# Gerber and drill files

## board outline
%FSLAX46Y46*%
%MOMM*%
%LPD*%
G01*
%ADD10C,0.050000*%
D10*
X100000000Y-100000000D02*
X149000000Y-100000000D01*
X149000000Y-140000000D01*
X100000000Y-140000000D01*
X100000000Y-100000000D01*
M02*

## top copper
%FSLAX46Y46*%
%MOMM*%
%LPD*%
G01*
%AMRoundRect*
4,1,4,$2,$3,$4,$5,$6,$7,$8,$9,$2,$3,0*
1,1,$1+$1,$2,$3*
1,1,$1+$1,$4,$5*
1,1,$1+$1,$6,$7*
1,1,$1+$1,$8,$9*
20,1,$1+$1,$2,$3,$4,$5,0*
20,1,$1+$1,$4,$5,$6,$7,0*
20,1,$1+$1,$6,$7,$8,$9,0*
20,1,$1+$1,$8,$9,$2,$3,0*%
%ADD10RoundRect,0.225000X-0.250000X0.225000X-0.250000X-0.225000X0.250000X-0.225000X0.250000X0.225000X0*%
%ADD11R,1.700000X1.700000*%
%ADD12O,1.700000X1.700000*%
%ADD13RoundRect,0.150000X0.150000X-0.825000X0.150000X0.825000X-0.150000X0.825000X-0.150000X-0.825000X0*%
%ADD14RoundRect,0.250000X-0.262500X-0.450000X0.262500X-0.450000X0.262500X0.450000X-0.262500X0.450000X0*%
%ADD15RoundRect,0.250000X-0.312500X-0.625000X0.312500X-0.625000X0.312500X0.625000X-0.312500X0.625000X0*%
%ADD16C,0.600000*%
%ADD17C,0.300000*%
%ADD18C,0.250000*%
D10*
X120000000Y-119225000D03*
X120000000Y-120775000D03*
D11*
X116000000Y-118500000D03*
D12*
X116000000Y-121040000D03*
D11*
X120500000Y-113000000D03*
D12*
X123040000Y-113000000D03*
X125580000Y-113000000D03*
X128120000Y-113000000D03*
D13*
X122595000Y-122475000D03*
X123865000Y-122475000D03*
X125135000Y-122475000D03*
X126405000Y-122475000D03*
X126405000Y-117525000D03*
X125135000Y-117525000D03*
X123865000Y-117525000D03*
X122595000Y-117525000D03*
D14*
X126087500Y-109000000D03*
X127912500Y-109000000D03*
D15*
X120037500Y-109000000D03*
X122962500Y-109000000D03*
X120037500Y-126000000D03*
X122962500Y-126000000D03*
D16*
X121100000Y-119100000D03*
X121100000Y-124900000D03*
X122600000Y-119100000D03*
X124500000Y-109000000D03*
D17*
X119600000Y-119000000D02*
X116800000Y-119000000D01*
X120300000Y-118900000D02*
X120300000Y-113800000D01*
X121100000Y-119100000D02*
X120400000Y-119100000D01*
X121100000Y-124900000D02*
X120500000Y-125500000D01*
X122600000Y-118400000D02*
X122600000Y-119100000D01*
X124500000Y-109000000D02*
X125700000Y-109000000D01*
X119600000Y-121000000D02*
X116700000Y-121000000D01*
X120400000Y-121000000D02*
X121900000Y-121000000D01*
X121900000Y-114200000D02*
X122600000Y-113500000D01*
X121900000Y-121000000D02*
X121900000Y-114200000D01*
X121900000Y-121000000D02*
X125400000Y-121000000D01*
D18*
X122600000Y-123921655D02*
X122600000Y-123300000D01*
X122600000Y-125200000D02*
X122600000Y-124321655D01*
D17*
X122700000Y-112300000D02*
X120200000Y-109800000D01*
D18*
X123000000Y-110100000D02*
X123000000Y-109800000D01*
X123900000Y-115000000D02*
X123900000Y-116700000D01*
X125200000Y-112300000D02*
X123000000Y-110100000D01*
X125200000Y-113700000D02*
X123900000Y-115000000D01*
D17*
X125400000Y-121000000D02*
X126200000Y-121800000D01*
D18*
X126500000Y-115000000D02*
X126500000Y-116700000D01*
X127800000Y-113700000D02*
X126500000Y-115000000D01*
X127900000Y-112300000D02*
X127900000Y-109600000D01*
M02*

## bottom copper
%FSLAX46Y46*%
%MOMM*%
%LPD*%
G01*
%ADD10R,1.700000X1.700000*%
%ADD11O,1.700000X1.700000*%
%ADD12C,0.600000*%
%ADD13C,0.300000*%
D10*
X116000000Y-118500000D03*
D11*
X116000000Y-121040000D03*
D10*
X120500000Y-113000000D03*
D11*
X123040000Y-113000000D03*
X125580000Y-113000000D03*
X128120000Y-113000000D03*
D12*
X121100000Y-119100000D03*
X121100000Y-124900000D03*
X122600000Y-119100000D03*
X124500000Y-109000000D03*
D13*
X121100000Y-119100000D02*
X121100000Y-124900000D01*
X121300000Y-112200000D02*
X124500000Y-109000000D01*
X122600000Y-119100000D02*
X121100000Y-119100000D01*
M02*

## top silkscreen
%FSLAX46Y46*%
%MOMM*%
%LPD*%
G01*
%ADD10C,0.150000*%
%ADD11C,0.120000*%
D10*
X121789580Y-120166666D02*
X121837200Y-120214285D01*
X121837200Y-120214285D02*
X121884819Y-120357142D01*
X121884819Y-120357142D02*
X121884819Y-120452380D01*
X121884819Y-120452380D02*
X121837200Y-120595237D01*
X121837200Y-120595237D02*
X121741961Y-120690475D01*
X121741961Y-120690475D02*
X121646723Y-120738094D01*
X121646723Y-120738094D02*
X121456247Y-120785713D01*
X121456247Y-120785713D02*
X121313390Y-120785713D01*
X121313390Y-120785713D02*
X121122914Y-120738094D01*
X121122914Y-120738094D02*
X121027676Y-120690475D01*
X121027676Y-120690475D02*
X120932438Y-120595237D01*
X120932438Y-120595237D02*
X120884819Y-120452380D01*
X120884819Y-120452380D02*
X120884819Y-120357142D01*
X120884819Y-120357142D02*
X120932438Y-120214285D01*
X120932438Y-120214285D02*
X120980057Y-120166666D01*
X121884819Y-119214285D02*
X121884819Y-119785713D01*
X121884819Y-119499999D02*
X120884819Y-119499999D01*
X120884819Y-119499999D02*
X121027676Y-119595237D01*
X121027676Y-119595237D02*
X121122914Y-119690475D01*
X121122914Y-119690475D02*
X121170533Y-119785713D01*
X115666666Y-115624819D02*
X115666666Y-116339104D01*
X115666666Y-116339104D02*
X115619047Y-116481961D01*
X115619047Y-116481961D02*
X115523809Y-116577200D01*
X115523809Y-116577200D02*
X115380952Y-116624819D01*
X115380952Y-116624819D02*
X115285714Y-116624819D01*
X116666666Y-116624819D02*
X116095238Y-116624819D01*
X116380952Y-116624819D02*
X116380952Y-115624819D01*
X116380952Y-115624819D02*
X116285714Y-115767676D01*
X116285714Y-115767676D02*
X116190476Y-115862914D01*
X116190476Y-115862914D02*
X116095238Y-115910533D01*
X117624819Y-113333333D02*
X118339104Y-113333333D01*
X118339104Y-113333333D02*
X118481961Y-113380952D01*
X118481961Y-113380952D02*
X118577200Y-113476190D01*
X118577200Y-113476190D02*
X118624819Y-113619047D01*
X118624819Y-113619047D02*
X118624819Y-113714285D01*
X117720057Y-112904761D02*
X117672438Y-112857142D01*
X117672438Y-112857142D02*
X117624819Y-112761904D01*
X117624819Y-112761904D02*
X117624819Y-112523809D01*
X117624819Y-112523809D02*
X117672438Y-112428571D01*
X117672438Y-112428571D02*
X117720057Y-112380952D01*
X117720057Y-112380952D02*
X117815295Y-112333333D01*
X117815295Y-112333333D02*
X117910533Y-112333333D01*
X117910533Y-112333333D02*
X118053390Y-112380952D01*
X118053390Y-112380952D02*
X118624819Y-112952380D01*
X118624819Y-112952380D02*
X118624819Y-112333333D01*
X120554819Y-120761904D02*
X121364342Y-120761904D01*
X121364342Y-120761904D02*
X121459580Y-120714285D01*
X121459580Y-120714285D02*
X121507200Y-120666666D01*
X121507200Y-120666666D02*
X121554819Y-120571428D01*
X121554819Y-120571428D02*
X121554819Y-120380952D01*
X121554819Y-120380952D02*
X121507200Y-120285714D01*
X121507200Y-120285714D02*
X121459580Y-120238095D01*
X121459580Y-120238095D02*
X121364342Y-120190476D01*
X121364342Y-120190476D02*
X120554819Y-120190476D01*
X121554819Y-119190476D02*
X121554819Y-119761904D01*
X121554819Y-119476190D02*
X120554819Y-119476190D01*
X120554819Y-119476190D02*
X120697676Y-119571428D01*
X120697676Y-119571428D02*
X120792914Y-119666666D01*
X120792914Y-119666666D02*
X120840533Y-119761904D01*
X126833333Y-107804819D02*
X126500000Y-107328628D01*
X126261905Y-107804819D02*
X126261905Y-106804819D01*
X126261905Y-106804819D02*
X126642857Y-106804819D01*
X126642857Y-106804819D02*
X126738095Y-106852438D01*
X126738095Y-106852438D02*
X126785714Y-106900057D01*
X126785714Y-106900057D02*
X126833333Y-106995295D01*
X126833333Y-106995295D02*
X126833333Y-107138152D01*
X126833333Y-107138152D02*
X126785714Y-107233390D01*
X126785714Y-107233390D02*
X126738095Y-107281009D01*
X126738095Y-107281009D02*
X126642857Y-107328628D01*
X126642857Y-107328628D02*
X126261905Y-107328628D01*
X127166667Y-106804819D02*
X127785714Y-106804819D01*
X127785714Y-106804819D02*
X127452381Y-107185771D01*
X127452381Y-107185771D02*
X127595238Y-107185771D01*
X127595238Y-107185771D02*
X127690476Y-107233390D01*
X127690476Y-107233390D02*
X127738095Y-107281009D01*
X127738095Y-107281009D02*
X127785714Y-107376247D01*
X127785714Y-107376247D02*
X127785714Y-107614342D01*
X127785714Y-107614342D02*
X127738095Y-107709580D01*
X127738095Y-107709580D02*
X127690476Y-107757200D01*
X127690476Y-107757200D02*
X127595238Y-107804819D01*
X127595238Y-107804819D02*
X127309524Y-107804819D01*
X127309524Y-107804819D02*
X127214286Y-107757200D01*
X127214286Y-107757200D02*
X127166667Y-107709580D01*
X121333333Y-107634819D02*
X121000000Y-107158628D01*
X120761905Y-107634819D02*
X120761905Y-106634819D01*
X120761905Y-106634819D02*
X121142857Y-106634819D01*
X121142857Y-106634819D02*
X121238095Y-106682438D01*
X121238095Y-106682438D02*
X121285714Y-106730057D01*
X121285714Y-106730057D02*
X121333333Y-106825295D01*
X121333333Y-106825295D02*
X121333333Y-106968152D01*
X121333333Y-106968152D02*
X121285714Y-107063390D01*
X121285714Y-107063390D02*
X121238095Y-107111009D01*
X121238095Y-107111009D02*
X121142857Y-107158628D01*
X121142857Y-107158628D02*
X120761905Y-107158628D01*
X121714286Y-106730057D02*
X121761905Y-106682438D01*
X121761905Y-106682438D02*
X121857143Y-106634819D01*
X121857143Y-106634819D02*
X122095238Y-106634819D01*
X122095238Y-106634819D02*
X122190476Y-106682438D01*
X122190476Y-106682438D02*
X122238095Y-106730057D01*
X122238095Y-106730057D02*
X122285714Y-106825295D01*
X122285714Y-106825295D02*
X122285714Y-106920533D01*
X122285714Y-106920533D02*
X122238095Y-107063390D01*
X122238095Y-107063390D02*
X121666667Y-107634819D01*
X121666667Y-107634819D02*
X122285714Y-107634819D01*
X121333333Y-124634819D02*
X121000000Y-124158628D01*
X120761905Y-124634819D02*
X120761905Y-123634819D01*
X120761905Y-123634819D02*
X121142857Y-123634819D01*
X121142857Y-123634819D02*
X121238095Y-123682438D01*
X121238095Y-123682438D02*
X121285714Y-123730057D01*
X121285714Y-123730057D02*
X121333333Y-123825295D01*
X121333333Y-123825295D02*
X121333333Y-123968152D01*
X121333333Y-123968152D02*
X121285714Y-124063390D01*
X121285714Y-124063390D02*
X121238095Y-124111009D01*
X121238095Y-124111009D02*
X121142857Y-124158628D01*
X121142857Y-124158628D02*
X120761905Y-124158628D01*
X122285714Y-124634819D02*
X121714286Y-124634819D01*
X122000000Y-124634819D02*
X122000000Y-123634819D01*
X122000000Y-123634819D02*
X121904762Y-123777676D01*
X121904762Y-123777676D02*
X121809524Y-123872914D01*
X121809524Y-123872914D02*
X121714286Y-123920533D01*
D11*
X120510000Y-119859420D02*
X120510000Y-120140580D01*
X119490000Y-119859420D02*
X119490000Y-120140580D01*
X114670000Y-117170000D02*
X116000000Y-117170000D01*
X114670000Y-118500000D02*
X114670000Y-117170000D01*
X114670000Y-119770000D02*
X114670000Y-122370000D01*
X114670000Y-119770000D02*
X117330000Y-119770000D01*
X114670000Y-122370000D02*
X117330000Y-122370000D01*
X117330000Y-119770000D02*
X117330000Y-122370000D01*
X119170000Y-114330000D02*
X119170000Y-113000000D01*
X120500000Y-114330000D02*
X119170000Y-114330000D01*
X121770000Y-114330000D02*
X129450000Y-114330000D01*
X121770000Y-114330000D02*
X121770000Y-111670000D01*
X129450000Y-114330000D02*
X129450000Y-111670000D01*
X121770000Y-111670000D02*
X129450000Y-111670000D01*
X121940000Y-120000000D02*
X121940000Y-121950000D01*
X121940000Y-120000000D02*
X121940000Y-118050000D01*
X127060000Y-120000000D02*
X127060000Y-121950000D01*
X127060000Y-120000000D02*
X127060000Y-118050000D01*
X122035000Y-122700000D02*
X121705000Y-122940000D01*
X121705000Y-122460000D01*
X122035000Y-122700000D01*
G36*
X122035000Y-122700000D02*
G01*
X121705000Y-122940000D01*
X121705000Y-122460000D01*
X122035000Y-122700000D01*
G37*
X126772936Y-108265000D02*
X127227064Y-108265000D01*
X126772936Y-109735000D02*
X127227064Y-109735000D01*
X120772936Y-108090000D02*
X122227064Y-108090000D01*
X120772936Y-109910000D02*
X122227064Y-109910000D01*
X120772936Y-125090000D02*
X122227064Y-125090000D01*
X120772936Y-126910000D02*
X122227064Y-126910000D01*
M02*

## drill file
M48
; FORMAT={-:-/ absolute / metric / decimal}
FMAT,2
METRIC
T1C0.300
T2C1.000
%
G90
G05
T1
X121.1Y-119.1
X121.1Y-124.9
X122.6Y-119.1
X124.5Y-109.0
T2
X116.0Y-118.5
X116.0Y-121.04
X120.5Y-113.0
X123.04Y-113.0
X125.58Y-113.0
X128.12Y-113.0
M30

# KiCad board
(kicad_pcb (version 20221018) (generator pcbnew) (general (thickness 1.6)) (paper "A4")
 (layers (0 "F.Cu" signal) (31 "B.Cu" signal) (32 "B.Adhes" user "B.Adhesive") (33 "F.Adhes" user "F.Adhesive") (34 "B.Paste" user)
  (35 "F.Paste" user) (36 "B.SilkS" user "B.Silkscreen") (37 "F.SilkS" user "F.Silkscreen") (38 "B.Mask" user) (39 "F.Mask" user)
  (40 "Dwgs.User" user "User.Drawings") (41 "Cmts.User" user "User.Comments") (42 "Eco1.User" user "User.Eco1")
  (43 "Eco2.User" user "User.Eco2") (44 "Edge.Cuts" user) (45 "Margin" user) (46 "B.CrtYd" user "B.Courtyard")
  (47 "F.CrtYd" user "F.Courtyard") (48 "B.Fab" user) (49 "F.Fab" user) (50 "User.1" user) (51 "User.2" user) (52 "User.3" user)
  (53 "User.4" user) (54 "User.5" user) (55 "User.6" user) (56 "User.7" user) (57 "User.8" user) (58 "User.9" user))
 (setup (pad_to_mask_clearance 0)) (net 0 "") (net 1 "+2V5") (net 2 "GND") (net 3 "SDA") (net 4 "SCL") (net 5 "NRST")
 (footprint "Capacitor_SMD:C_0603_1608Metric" (layer "F.Cu") (at 120 120 -90)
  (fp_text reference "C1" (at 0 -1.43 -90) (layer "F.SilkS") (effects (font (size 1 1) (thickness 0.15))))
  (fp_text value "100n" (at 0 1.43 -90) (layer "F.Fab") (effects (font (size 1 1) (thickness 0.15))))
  (fp_line (start -0.14058 -0.51) (end 0.14058 -0.51) (stroke (width 0.12) (type solid)) (layer "F.SilkS"))
  (fp_line (start -0.14058 0.51) (end 0.14058 0.51) (stroke (width 0.12) (type solid)) (layer "F.SilkS"))
  (pad "1" smd roundrect (at -0.775 0 270) (size 0.9 0.95) (layers "F.Cu" "F.Paste" "F.Mask") (roundrect_rratio 0.25) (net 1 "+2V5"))
  (pad "2" smd roundrect (at 0.775 0 270) (size 0.9 0.95) (layers "F.Cu" "F.Paste" "F.Mask") (roundrect_rratio 0.25) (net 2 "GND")))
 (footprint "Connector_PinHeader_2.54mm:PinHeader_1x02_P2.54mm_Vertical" (layer "F.Cu") (at 116 118.5)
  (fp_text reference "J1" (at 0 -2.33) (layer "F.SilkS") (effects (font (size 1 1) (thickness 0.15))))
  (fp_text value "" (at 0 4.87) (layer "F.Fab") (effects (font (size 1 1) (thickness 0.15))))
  (fp_line (start -1.33 -1.33) (end 0 -1.33) (stroke (width 0.12) (type solid)) (layer "F.SilkS"))
  (fp_line (start -1.33 0) (end -1.33 -1.33) (stroke (width 0.12) (type solid)) (layer "F.SilkS"))
  (fp_line (start -1.33 1.27) (end -1.33 3.87) (stroke (width 0.12) (type solid)) (layer "F.SilkS"))
  (fp_line (start -1.33 1.27) (end 1.33 1.27) (stroke (width 0.12) (type solid)) (layer "F.SilkS"))
  (fp_line (start -1.33 3.87) (end 1.33 3.87) (stroke (width 0.12) (type solid)) (layer "F.SilkS"))
  (fp_line (start 1.33 1.27) (end 1.33 3.87) (stroke (width 0.12) (type solid)) (layer "F.SilkS"))
  (pad "1" thru_hole rect (at 0 0) (size 1.7 1.7) (drill 1) (layers "*.Cu" "*.Mask") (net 1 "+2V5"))
  (pad "2" thru_hole oval (at 0 2.54) (size 1.7 1.7) (drill 1) (layers "*.Cu" "*.Mask") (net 2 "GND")))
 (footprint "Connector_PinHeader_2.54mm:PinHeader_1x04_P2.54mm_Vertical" (layer "F.Cu") (at 120.5 113 90)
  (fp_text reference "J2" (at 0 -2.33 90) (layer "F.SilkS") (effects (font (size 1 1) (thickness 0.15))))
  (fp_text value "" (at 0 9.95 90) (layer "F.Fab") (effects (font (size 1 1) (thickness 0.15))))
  (fp_line (start -1.33 -1.33) (end 0 -1.33) (stroke (width 0.12) (type solid)) (layer "F.SilkS"))
  (fp_line (start -1.33 0) (end -1.33 -1.33) (stroke (width 0.12) (type solid)) (layer "F.SilkS"))
  (fp_line (start -1.33 1.27) (end -1.33 8.95) (stroke (width 0.12) (type solid)) (layer "F.SilkS"))
  (fp_line (start -1.33 1.27) (end 1.33 1.27) (stroke (width 0.12) (type solid)) (layer "F.SilkS"))
  (fp_line (start -1.33 8.95) (end 1.33 8.95) (stroke (width 0.12) (type solid)) (layer "F.SilkS"))
  (fp_line (start 1.33 1.27) (end 1.33 8.95) (stroke (width 0.12) (type solid)) (layer "F.SilkS"))
  (pad "1" thru_hole rect (at 0 0 90) (size 1.7 1.7) (drill 1) (layers "*.Cu" "*.Mask") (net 1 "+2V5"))
  (pad "2" thru_hole oval (at 0 2.54 90) (size 1.7 1.7) (drill 1) (layers "*.Cu" "*.Mask") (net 2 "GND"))
  (pad "3" thru_hole oval (at 0 5.08 90) (size 1.7 1.7) (drill 1) (layers "*.Cu" "*.Mask") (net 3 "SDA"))
  (pad "4" thru_hole oval (at 0 7.62 90) (size 1.7 1.7) (drill 1) (layers "*.Cu" "*.Mask") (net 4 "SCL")))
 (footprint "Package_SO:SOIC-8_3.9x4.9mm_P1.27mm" (layer "F.Cu") (at 124.5 120 90)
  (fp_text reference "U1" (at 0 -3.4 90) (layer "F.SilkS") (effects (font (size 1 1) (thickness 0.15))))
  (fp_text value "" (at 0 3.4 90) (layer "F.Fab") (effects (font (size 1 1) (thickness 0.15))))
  (fp_line (start 0 -2.56) (end -1.95 -2.56) (stroke (width 0.12) (type solid)) (layer "F.SilkS"))
  (fp_line (start 0 -2.56) (end 1.95 -2.56) (stroke (width 0.12) (type solid)) (layer "F.SilkS"))
  (fp_line (start 0 2.56) (end -1.95 2.56) (stroke (width 0.12) (type solid)) (layer "F.SilkS"))
  (fp_line (start 0 2.56) (end 1.95 2.56) (stroke (width 0.12) (type solid)) (layer "F.SilkS"))
  (fp_poly
   (pts (xy -2.7 -2.465) (xy -2.94 -2.795) (xy -2.46 -2.795) (xy -2.7 -2.465)) (stroke (width 0.12) (type solid)) (fill solid)
   (layer "F.SilkS"))
  (pad "1" smd roundrect (at -2.475 -1.905 90) (size 1.95 0.6) (layers "F.Cu" "F.Paste" "F.Mask") (roundrect_rratio 0.25) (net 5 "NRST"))
  (pad "2" smd roundrect (at -2.475 -0.635 90) (size 1.95 0.6) (layers "F.Cu" "F.Paste" "F.Mask") (roundrect_rratio 0.25))
  (pad "3" smd roundrect (at -2.475 0.635 90) (size 1.95 0.6) (layers "F.Cu" "F.Paste" "F.Mask") (roundrect_rratio 0.25))
  (pad "4" smd roundrect (at -2.475 1.905 90) (size 1.95 0.6) (layers "F.Cu" "F.Paste" "F.Mask") (roundrect_rratio 0.25) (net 2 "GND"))
  (pad "5" smd roundrect (at 2.475 1.905 90) (size 1.95 0.6) (layers "F.Cu" "F.Paste" "F.Mask") (roundrect_rratio 0.25) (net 4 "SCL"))
  (pad "6" smd roundrect (at 2.475 0.635 90) (size 1.95 0.6) (layers "F.Cu" "F.Paste" "F.Mask") (roundrect_rratio 0.25))
  (pad "7" smd roundrect (at 2.475 -0.635 90) (size 1.95 0.6) (layers "F.Cu" "F.Paste" "F.Mask") (roundrect_rratio 0.25) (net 3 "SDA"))
  (pad "8" smd roundrect (at 2.475 -1.905 90) (size 1.95 0.6) (layers "F.Cu" "F.Paste" "F.Mask") (roundrect_rratio 0.25) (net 1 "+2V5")))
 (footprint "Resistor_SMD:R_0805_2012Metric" (layer "F.Cu") (at 127 109)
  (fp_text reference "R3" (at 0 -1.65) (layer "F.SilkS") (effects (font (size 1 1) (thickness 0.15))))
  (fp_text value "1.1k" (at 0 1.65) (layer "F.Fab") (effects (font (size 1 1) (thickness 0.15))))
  (fp_line (start -0.227064 -0.735) (end 0.227064 -0.735) (stroke (width 0.12) (type solid)) (layer "F.SilkS"))
  (fp_line (start -0.227064 0.735) (end 0.227064 0.735) (stroke (width 0.12) (type solid)) (layer "F.SilkS"))
  (pad "1" smd roundrect (at -0.9125 0) (size 1.025 1.4) (layers "F.Cu" "F.Paste" "F.Mask") (roundrect_rratio 0.243902) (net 1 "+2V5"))
  (pad "2" smd roundrect (at 0.9125 0) (size 1.025 1.4) (layers "F.Cu" "F.Paste" "F.Mask") (roundrect_rratio 0.243902) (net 4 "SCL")))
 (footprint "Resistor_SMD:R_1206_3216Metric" (layer "F.Cu") (at 121.5 109)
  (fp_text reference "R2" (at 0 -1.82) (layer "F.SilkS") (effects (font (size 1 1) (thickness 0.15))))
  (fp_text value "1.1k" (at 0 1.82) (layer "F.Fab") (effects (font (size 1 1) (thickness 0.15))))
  (fp_line (start -0.727064 -0.91) (end 0.727064 -0.91) (stroke (width 0.12) (type solid)) (layer "F.SilkS"))
  (fp_line (start -0.727064 0.91) (end 0.727064 0.91) (stroke (width 0.12) (type solid)) (layer "F.SilkS"))
  (pad "1" smd roundrect (at -1.4625 0) (size 1.125 1.75) (layers "F.Cu" "F.Paste" "F.Mask") (roundrect_rratio 0.222222) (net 2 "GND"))
  (pad "2" smd roundrect (at 1.4625 0) (size 1.125 1.75) (layers "F.Cu" "F.Paste" "F.Mask") (roundrect_rratio 0.222222) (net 3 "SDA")))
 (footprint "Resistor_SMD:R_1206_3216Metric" (layer "F.Cu") (at 121.5 126)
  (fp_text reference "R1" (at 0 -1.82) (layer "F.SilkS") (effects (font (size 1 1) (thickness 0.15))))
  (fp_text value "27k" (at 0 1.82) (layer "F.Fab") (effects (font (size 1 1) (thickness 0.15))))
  (fp_line (start -0.727064 -0.91) (end 0.727064 -0.91) (stroke (width 0.12) (type solid)) (layer "F.SilkS"))
  (fp_line (start -0.727064 0.91) (end 0.727064 0.91) (stroke (width 0.12) (type solid)) (layer "F.SilkS"))
  (pad "1" smd roundrect (at -1.4625 0) (size 1.125 1.75) (layers "F.Cu" "F.Paste" "F.Mask") (roundrect_rratio 0.222222) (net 1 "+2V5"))
  (pad "2" smd roundrect (at 1.4625 0) (size 1.125 1.75) (layers "F.Cu" "F.Paste" "F.Mask") (roundrect_rratio 0.222222) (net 5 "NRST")))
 (gr_rect (start 100 100) (end 149 140) (stroke (width 0.05) (type default)) (fill none) (layer "Edge.Cuts"))
 (segment (start 119.6 119) (end 116.8 119) (width 0.3) (layer "F.Cu") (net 1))
 (segment (start 120.3 118.9) (end 120.3 113.8) (width 0.3) (layer "F.Cu") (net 1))
 (segment (start 121.1 119.1) (end 120.4 119.1) (width 0.3) (layer "F.Cu") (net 1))
 (segment (start 121.1 124.9) (end 120.5 125.5) (width 0.3) (layer "F.Cu") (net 1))
 (segment (start 122.6 118.4) (end 122.6 119.1) (width 0.3) (layer "F.Cu") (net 1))
 (segment (start 124.5 109) (end 125.7 109) (width 0.3) (layer "F.Cu") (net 1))
 (via (at 121.1 119.1) (size 0.6) (drill 0.3) (layers "F.Cu" "B.Cu") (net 1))
 (via (at 121.1 124.9) (size 0.6) (drill 0.3) (layers "F.Cu" "B.Cu") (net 1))
 (via (at 122.6 119.1) (size 0.6) (drill 0.3) (layers "F.Cu" "B.Cu") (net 1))
 (via (at 124.5 109) (size 0.6) (drill 0.3) (layers "F.Cu" "B.Cu") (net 1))
 (segment (start 119.6 121) (end 116.7 121) (width 0.3) (layer "F.Cu") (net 2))
 (segment (start 120.4 121) (end 121.9 121) (width 0.3) (layer "F.Cu") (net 2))
 (segment (start 121.1 119.1) (end 121.1 124.9) (width 0.3) (layer "B.Cu") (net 1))
 (segment (start 121.3 112.2) (end 124.5 109) (width 0.3) (layer "B.Cu") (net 1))
 (segment (start 121.9 114.2) (end 122.6 113.5) (width 0.3) (layer "F.Cu") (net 2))
 (segment (start 121.9 121) (end 121.9 114.2) (width 0.3) (layer "F.Cu") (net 2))
 (segment (start 121.9 121) (end 125.4 121) (width 0.3) (layer "F.Cu") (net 2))
 (segment (start 122.6 119.1) (end 121.1 119.1) (width 0.3) (layer "B.Cu") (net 1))
 (segment (start 122.6 123.921655) (end 122.6 123.3) (width 0.25) (layer "F.Cu") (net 5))
 (segment (start 122.6 125.2) (end 122.6 124.321655) (width 0.25) (layer "F.Cu") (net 5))
 (segment (start 122.7 112.3) (end 120.2 109.8) (width 0.3) (layer "F.Cu") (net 2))
 (segment (start 123 110.1) (end 123 109.8) (width 0.25) (layer "F.Cu") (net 3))
 (segment (start 123.9 115) (end 123.9 116.7) (width 0.25) (layer "F.Cu") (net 3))
 (segment (start 125.2 112.3) (end 123 110.1) (width 0.25) (layer "F.Cu") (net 3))
 (segment (start 125.2 113.7) (end 123.9 115) (width 0.25) (layer "F.Cu") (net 3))
 (segment (start 125.4 121) (end 126.2 121.8) (width 0.3) (layer "F.Cu") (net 2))
 (segment (start 126.5 115) (end 126.5 116.7) (width 0.25) (layer "F.Cu") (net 4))
 (segment (start 127.8 113.7) (end 126.5 115) (width 0.25) (layer "F.Cu") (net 4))
 (segment (start 127.9 112.3) (end 127.9 109.6) (width 0.25) (layer "F.Cu") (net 4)))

